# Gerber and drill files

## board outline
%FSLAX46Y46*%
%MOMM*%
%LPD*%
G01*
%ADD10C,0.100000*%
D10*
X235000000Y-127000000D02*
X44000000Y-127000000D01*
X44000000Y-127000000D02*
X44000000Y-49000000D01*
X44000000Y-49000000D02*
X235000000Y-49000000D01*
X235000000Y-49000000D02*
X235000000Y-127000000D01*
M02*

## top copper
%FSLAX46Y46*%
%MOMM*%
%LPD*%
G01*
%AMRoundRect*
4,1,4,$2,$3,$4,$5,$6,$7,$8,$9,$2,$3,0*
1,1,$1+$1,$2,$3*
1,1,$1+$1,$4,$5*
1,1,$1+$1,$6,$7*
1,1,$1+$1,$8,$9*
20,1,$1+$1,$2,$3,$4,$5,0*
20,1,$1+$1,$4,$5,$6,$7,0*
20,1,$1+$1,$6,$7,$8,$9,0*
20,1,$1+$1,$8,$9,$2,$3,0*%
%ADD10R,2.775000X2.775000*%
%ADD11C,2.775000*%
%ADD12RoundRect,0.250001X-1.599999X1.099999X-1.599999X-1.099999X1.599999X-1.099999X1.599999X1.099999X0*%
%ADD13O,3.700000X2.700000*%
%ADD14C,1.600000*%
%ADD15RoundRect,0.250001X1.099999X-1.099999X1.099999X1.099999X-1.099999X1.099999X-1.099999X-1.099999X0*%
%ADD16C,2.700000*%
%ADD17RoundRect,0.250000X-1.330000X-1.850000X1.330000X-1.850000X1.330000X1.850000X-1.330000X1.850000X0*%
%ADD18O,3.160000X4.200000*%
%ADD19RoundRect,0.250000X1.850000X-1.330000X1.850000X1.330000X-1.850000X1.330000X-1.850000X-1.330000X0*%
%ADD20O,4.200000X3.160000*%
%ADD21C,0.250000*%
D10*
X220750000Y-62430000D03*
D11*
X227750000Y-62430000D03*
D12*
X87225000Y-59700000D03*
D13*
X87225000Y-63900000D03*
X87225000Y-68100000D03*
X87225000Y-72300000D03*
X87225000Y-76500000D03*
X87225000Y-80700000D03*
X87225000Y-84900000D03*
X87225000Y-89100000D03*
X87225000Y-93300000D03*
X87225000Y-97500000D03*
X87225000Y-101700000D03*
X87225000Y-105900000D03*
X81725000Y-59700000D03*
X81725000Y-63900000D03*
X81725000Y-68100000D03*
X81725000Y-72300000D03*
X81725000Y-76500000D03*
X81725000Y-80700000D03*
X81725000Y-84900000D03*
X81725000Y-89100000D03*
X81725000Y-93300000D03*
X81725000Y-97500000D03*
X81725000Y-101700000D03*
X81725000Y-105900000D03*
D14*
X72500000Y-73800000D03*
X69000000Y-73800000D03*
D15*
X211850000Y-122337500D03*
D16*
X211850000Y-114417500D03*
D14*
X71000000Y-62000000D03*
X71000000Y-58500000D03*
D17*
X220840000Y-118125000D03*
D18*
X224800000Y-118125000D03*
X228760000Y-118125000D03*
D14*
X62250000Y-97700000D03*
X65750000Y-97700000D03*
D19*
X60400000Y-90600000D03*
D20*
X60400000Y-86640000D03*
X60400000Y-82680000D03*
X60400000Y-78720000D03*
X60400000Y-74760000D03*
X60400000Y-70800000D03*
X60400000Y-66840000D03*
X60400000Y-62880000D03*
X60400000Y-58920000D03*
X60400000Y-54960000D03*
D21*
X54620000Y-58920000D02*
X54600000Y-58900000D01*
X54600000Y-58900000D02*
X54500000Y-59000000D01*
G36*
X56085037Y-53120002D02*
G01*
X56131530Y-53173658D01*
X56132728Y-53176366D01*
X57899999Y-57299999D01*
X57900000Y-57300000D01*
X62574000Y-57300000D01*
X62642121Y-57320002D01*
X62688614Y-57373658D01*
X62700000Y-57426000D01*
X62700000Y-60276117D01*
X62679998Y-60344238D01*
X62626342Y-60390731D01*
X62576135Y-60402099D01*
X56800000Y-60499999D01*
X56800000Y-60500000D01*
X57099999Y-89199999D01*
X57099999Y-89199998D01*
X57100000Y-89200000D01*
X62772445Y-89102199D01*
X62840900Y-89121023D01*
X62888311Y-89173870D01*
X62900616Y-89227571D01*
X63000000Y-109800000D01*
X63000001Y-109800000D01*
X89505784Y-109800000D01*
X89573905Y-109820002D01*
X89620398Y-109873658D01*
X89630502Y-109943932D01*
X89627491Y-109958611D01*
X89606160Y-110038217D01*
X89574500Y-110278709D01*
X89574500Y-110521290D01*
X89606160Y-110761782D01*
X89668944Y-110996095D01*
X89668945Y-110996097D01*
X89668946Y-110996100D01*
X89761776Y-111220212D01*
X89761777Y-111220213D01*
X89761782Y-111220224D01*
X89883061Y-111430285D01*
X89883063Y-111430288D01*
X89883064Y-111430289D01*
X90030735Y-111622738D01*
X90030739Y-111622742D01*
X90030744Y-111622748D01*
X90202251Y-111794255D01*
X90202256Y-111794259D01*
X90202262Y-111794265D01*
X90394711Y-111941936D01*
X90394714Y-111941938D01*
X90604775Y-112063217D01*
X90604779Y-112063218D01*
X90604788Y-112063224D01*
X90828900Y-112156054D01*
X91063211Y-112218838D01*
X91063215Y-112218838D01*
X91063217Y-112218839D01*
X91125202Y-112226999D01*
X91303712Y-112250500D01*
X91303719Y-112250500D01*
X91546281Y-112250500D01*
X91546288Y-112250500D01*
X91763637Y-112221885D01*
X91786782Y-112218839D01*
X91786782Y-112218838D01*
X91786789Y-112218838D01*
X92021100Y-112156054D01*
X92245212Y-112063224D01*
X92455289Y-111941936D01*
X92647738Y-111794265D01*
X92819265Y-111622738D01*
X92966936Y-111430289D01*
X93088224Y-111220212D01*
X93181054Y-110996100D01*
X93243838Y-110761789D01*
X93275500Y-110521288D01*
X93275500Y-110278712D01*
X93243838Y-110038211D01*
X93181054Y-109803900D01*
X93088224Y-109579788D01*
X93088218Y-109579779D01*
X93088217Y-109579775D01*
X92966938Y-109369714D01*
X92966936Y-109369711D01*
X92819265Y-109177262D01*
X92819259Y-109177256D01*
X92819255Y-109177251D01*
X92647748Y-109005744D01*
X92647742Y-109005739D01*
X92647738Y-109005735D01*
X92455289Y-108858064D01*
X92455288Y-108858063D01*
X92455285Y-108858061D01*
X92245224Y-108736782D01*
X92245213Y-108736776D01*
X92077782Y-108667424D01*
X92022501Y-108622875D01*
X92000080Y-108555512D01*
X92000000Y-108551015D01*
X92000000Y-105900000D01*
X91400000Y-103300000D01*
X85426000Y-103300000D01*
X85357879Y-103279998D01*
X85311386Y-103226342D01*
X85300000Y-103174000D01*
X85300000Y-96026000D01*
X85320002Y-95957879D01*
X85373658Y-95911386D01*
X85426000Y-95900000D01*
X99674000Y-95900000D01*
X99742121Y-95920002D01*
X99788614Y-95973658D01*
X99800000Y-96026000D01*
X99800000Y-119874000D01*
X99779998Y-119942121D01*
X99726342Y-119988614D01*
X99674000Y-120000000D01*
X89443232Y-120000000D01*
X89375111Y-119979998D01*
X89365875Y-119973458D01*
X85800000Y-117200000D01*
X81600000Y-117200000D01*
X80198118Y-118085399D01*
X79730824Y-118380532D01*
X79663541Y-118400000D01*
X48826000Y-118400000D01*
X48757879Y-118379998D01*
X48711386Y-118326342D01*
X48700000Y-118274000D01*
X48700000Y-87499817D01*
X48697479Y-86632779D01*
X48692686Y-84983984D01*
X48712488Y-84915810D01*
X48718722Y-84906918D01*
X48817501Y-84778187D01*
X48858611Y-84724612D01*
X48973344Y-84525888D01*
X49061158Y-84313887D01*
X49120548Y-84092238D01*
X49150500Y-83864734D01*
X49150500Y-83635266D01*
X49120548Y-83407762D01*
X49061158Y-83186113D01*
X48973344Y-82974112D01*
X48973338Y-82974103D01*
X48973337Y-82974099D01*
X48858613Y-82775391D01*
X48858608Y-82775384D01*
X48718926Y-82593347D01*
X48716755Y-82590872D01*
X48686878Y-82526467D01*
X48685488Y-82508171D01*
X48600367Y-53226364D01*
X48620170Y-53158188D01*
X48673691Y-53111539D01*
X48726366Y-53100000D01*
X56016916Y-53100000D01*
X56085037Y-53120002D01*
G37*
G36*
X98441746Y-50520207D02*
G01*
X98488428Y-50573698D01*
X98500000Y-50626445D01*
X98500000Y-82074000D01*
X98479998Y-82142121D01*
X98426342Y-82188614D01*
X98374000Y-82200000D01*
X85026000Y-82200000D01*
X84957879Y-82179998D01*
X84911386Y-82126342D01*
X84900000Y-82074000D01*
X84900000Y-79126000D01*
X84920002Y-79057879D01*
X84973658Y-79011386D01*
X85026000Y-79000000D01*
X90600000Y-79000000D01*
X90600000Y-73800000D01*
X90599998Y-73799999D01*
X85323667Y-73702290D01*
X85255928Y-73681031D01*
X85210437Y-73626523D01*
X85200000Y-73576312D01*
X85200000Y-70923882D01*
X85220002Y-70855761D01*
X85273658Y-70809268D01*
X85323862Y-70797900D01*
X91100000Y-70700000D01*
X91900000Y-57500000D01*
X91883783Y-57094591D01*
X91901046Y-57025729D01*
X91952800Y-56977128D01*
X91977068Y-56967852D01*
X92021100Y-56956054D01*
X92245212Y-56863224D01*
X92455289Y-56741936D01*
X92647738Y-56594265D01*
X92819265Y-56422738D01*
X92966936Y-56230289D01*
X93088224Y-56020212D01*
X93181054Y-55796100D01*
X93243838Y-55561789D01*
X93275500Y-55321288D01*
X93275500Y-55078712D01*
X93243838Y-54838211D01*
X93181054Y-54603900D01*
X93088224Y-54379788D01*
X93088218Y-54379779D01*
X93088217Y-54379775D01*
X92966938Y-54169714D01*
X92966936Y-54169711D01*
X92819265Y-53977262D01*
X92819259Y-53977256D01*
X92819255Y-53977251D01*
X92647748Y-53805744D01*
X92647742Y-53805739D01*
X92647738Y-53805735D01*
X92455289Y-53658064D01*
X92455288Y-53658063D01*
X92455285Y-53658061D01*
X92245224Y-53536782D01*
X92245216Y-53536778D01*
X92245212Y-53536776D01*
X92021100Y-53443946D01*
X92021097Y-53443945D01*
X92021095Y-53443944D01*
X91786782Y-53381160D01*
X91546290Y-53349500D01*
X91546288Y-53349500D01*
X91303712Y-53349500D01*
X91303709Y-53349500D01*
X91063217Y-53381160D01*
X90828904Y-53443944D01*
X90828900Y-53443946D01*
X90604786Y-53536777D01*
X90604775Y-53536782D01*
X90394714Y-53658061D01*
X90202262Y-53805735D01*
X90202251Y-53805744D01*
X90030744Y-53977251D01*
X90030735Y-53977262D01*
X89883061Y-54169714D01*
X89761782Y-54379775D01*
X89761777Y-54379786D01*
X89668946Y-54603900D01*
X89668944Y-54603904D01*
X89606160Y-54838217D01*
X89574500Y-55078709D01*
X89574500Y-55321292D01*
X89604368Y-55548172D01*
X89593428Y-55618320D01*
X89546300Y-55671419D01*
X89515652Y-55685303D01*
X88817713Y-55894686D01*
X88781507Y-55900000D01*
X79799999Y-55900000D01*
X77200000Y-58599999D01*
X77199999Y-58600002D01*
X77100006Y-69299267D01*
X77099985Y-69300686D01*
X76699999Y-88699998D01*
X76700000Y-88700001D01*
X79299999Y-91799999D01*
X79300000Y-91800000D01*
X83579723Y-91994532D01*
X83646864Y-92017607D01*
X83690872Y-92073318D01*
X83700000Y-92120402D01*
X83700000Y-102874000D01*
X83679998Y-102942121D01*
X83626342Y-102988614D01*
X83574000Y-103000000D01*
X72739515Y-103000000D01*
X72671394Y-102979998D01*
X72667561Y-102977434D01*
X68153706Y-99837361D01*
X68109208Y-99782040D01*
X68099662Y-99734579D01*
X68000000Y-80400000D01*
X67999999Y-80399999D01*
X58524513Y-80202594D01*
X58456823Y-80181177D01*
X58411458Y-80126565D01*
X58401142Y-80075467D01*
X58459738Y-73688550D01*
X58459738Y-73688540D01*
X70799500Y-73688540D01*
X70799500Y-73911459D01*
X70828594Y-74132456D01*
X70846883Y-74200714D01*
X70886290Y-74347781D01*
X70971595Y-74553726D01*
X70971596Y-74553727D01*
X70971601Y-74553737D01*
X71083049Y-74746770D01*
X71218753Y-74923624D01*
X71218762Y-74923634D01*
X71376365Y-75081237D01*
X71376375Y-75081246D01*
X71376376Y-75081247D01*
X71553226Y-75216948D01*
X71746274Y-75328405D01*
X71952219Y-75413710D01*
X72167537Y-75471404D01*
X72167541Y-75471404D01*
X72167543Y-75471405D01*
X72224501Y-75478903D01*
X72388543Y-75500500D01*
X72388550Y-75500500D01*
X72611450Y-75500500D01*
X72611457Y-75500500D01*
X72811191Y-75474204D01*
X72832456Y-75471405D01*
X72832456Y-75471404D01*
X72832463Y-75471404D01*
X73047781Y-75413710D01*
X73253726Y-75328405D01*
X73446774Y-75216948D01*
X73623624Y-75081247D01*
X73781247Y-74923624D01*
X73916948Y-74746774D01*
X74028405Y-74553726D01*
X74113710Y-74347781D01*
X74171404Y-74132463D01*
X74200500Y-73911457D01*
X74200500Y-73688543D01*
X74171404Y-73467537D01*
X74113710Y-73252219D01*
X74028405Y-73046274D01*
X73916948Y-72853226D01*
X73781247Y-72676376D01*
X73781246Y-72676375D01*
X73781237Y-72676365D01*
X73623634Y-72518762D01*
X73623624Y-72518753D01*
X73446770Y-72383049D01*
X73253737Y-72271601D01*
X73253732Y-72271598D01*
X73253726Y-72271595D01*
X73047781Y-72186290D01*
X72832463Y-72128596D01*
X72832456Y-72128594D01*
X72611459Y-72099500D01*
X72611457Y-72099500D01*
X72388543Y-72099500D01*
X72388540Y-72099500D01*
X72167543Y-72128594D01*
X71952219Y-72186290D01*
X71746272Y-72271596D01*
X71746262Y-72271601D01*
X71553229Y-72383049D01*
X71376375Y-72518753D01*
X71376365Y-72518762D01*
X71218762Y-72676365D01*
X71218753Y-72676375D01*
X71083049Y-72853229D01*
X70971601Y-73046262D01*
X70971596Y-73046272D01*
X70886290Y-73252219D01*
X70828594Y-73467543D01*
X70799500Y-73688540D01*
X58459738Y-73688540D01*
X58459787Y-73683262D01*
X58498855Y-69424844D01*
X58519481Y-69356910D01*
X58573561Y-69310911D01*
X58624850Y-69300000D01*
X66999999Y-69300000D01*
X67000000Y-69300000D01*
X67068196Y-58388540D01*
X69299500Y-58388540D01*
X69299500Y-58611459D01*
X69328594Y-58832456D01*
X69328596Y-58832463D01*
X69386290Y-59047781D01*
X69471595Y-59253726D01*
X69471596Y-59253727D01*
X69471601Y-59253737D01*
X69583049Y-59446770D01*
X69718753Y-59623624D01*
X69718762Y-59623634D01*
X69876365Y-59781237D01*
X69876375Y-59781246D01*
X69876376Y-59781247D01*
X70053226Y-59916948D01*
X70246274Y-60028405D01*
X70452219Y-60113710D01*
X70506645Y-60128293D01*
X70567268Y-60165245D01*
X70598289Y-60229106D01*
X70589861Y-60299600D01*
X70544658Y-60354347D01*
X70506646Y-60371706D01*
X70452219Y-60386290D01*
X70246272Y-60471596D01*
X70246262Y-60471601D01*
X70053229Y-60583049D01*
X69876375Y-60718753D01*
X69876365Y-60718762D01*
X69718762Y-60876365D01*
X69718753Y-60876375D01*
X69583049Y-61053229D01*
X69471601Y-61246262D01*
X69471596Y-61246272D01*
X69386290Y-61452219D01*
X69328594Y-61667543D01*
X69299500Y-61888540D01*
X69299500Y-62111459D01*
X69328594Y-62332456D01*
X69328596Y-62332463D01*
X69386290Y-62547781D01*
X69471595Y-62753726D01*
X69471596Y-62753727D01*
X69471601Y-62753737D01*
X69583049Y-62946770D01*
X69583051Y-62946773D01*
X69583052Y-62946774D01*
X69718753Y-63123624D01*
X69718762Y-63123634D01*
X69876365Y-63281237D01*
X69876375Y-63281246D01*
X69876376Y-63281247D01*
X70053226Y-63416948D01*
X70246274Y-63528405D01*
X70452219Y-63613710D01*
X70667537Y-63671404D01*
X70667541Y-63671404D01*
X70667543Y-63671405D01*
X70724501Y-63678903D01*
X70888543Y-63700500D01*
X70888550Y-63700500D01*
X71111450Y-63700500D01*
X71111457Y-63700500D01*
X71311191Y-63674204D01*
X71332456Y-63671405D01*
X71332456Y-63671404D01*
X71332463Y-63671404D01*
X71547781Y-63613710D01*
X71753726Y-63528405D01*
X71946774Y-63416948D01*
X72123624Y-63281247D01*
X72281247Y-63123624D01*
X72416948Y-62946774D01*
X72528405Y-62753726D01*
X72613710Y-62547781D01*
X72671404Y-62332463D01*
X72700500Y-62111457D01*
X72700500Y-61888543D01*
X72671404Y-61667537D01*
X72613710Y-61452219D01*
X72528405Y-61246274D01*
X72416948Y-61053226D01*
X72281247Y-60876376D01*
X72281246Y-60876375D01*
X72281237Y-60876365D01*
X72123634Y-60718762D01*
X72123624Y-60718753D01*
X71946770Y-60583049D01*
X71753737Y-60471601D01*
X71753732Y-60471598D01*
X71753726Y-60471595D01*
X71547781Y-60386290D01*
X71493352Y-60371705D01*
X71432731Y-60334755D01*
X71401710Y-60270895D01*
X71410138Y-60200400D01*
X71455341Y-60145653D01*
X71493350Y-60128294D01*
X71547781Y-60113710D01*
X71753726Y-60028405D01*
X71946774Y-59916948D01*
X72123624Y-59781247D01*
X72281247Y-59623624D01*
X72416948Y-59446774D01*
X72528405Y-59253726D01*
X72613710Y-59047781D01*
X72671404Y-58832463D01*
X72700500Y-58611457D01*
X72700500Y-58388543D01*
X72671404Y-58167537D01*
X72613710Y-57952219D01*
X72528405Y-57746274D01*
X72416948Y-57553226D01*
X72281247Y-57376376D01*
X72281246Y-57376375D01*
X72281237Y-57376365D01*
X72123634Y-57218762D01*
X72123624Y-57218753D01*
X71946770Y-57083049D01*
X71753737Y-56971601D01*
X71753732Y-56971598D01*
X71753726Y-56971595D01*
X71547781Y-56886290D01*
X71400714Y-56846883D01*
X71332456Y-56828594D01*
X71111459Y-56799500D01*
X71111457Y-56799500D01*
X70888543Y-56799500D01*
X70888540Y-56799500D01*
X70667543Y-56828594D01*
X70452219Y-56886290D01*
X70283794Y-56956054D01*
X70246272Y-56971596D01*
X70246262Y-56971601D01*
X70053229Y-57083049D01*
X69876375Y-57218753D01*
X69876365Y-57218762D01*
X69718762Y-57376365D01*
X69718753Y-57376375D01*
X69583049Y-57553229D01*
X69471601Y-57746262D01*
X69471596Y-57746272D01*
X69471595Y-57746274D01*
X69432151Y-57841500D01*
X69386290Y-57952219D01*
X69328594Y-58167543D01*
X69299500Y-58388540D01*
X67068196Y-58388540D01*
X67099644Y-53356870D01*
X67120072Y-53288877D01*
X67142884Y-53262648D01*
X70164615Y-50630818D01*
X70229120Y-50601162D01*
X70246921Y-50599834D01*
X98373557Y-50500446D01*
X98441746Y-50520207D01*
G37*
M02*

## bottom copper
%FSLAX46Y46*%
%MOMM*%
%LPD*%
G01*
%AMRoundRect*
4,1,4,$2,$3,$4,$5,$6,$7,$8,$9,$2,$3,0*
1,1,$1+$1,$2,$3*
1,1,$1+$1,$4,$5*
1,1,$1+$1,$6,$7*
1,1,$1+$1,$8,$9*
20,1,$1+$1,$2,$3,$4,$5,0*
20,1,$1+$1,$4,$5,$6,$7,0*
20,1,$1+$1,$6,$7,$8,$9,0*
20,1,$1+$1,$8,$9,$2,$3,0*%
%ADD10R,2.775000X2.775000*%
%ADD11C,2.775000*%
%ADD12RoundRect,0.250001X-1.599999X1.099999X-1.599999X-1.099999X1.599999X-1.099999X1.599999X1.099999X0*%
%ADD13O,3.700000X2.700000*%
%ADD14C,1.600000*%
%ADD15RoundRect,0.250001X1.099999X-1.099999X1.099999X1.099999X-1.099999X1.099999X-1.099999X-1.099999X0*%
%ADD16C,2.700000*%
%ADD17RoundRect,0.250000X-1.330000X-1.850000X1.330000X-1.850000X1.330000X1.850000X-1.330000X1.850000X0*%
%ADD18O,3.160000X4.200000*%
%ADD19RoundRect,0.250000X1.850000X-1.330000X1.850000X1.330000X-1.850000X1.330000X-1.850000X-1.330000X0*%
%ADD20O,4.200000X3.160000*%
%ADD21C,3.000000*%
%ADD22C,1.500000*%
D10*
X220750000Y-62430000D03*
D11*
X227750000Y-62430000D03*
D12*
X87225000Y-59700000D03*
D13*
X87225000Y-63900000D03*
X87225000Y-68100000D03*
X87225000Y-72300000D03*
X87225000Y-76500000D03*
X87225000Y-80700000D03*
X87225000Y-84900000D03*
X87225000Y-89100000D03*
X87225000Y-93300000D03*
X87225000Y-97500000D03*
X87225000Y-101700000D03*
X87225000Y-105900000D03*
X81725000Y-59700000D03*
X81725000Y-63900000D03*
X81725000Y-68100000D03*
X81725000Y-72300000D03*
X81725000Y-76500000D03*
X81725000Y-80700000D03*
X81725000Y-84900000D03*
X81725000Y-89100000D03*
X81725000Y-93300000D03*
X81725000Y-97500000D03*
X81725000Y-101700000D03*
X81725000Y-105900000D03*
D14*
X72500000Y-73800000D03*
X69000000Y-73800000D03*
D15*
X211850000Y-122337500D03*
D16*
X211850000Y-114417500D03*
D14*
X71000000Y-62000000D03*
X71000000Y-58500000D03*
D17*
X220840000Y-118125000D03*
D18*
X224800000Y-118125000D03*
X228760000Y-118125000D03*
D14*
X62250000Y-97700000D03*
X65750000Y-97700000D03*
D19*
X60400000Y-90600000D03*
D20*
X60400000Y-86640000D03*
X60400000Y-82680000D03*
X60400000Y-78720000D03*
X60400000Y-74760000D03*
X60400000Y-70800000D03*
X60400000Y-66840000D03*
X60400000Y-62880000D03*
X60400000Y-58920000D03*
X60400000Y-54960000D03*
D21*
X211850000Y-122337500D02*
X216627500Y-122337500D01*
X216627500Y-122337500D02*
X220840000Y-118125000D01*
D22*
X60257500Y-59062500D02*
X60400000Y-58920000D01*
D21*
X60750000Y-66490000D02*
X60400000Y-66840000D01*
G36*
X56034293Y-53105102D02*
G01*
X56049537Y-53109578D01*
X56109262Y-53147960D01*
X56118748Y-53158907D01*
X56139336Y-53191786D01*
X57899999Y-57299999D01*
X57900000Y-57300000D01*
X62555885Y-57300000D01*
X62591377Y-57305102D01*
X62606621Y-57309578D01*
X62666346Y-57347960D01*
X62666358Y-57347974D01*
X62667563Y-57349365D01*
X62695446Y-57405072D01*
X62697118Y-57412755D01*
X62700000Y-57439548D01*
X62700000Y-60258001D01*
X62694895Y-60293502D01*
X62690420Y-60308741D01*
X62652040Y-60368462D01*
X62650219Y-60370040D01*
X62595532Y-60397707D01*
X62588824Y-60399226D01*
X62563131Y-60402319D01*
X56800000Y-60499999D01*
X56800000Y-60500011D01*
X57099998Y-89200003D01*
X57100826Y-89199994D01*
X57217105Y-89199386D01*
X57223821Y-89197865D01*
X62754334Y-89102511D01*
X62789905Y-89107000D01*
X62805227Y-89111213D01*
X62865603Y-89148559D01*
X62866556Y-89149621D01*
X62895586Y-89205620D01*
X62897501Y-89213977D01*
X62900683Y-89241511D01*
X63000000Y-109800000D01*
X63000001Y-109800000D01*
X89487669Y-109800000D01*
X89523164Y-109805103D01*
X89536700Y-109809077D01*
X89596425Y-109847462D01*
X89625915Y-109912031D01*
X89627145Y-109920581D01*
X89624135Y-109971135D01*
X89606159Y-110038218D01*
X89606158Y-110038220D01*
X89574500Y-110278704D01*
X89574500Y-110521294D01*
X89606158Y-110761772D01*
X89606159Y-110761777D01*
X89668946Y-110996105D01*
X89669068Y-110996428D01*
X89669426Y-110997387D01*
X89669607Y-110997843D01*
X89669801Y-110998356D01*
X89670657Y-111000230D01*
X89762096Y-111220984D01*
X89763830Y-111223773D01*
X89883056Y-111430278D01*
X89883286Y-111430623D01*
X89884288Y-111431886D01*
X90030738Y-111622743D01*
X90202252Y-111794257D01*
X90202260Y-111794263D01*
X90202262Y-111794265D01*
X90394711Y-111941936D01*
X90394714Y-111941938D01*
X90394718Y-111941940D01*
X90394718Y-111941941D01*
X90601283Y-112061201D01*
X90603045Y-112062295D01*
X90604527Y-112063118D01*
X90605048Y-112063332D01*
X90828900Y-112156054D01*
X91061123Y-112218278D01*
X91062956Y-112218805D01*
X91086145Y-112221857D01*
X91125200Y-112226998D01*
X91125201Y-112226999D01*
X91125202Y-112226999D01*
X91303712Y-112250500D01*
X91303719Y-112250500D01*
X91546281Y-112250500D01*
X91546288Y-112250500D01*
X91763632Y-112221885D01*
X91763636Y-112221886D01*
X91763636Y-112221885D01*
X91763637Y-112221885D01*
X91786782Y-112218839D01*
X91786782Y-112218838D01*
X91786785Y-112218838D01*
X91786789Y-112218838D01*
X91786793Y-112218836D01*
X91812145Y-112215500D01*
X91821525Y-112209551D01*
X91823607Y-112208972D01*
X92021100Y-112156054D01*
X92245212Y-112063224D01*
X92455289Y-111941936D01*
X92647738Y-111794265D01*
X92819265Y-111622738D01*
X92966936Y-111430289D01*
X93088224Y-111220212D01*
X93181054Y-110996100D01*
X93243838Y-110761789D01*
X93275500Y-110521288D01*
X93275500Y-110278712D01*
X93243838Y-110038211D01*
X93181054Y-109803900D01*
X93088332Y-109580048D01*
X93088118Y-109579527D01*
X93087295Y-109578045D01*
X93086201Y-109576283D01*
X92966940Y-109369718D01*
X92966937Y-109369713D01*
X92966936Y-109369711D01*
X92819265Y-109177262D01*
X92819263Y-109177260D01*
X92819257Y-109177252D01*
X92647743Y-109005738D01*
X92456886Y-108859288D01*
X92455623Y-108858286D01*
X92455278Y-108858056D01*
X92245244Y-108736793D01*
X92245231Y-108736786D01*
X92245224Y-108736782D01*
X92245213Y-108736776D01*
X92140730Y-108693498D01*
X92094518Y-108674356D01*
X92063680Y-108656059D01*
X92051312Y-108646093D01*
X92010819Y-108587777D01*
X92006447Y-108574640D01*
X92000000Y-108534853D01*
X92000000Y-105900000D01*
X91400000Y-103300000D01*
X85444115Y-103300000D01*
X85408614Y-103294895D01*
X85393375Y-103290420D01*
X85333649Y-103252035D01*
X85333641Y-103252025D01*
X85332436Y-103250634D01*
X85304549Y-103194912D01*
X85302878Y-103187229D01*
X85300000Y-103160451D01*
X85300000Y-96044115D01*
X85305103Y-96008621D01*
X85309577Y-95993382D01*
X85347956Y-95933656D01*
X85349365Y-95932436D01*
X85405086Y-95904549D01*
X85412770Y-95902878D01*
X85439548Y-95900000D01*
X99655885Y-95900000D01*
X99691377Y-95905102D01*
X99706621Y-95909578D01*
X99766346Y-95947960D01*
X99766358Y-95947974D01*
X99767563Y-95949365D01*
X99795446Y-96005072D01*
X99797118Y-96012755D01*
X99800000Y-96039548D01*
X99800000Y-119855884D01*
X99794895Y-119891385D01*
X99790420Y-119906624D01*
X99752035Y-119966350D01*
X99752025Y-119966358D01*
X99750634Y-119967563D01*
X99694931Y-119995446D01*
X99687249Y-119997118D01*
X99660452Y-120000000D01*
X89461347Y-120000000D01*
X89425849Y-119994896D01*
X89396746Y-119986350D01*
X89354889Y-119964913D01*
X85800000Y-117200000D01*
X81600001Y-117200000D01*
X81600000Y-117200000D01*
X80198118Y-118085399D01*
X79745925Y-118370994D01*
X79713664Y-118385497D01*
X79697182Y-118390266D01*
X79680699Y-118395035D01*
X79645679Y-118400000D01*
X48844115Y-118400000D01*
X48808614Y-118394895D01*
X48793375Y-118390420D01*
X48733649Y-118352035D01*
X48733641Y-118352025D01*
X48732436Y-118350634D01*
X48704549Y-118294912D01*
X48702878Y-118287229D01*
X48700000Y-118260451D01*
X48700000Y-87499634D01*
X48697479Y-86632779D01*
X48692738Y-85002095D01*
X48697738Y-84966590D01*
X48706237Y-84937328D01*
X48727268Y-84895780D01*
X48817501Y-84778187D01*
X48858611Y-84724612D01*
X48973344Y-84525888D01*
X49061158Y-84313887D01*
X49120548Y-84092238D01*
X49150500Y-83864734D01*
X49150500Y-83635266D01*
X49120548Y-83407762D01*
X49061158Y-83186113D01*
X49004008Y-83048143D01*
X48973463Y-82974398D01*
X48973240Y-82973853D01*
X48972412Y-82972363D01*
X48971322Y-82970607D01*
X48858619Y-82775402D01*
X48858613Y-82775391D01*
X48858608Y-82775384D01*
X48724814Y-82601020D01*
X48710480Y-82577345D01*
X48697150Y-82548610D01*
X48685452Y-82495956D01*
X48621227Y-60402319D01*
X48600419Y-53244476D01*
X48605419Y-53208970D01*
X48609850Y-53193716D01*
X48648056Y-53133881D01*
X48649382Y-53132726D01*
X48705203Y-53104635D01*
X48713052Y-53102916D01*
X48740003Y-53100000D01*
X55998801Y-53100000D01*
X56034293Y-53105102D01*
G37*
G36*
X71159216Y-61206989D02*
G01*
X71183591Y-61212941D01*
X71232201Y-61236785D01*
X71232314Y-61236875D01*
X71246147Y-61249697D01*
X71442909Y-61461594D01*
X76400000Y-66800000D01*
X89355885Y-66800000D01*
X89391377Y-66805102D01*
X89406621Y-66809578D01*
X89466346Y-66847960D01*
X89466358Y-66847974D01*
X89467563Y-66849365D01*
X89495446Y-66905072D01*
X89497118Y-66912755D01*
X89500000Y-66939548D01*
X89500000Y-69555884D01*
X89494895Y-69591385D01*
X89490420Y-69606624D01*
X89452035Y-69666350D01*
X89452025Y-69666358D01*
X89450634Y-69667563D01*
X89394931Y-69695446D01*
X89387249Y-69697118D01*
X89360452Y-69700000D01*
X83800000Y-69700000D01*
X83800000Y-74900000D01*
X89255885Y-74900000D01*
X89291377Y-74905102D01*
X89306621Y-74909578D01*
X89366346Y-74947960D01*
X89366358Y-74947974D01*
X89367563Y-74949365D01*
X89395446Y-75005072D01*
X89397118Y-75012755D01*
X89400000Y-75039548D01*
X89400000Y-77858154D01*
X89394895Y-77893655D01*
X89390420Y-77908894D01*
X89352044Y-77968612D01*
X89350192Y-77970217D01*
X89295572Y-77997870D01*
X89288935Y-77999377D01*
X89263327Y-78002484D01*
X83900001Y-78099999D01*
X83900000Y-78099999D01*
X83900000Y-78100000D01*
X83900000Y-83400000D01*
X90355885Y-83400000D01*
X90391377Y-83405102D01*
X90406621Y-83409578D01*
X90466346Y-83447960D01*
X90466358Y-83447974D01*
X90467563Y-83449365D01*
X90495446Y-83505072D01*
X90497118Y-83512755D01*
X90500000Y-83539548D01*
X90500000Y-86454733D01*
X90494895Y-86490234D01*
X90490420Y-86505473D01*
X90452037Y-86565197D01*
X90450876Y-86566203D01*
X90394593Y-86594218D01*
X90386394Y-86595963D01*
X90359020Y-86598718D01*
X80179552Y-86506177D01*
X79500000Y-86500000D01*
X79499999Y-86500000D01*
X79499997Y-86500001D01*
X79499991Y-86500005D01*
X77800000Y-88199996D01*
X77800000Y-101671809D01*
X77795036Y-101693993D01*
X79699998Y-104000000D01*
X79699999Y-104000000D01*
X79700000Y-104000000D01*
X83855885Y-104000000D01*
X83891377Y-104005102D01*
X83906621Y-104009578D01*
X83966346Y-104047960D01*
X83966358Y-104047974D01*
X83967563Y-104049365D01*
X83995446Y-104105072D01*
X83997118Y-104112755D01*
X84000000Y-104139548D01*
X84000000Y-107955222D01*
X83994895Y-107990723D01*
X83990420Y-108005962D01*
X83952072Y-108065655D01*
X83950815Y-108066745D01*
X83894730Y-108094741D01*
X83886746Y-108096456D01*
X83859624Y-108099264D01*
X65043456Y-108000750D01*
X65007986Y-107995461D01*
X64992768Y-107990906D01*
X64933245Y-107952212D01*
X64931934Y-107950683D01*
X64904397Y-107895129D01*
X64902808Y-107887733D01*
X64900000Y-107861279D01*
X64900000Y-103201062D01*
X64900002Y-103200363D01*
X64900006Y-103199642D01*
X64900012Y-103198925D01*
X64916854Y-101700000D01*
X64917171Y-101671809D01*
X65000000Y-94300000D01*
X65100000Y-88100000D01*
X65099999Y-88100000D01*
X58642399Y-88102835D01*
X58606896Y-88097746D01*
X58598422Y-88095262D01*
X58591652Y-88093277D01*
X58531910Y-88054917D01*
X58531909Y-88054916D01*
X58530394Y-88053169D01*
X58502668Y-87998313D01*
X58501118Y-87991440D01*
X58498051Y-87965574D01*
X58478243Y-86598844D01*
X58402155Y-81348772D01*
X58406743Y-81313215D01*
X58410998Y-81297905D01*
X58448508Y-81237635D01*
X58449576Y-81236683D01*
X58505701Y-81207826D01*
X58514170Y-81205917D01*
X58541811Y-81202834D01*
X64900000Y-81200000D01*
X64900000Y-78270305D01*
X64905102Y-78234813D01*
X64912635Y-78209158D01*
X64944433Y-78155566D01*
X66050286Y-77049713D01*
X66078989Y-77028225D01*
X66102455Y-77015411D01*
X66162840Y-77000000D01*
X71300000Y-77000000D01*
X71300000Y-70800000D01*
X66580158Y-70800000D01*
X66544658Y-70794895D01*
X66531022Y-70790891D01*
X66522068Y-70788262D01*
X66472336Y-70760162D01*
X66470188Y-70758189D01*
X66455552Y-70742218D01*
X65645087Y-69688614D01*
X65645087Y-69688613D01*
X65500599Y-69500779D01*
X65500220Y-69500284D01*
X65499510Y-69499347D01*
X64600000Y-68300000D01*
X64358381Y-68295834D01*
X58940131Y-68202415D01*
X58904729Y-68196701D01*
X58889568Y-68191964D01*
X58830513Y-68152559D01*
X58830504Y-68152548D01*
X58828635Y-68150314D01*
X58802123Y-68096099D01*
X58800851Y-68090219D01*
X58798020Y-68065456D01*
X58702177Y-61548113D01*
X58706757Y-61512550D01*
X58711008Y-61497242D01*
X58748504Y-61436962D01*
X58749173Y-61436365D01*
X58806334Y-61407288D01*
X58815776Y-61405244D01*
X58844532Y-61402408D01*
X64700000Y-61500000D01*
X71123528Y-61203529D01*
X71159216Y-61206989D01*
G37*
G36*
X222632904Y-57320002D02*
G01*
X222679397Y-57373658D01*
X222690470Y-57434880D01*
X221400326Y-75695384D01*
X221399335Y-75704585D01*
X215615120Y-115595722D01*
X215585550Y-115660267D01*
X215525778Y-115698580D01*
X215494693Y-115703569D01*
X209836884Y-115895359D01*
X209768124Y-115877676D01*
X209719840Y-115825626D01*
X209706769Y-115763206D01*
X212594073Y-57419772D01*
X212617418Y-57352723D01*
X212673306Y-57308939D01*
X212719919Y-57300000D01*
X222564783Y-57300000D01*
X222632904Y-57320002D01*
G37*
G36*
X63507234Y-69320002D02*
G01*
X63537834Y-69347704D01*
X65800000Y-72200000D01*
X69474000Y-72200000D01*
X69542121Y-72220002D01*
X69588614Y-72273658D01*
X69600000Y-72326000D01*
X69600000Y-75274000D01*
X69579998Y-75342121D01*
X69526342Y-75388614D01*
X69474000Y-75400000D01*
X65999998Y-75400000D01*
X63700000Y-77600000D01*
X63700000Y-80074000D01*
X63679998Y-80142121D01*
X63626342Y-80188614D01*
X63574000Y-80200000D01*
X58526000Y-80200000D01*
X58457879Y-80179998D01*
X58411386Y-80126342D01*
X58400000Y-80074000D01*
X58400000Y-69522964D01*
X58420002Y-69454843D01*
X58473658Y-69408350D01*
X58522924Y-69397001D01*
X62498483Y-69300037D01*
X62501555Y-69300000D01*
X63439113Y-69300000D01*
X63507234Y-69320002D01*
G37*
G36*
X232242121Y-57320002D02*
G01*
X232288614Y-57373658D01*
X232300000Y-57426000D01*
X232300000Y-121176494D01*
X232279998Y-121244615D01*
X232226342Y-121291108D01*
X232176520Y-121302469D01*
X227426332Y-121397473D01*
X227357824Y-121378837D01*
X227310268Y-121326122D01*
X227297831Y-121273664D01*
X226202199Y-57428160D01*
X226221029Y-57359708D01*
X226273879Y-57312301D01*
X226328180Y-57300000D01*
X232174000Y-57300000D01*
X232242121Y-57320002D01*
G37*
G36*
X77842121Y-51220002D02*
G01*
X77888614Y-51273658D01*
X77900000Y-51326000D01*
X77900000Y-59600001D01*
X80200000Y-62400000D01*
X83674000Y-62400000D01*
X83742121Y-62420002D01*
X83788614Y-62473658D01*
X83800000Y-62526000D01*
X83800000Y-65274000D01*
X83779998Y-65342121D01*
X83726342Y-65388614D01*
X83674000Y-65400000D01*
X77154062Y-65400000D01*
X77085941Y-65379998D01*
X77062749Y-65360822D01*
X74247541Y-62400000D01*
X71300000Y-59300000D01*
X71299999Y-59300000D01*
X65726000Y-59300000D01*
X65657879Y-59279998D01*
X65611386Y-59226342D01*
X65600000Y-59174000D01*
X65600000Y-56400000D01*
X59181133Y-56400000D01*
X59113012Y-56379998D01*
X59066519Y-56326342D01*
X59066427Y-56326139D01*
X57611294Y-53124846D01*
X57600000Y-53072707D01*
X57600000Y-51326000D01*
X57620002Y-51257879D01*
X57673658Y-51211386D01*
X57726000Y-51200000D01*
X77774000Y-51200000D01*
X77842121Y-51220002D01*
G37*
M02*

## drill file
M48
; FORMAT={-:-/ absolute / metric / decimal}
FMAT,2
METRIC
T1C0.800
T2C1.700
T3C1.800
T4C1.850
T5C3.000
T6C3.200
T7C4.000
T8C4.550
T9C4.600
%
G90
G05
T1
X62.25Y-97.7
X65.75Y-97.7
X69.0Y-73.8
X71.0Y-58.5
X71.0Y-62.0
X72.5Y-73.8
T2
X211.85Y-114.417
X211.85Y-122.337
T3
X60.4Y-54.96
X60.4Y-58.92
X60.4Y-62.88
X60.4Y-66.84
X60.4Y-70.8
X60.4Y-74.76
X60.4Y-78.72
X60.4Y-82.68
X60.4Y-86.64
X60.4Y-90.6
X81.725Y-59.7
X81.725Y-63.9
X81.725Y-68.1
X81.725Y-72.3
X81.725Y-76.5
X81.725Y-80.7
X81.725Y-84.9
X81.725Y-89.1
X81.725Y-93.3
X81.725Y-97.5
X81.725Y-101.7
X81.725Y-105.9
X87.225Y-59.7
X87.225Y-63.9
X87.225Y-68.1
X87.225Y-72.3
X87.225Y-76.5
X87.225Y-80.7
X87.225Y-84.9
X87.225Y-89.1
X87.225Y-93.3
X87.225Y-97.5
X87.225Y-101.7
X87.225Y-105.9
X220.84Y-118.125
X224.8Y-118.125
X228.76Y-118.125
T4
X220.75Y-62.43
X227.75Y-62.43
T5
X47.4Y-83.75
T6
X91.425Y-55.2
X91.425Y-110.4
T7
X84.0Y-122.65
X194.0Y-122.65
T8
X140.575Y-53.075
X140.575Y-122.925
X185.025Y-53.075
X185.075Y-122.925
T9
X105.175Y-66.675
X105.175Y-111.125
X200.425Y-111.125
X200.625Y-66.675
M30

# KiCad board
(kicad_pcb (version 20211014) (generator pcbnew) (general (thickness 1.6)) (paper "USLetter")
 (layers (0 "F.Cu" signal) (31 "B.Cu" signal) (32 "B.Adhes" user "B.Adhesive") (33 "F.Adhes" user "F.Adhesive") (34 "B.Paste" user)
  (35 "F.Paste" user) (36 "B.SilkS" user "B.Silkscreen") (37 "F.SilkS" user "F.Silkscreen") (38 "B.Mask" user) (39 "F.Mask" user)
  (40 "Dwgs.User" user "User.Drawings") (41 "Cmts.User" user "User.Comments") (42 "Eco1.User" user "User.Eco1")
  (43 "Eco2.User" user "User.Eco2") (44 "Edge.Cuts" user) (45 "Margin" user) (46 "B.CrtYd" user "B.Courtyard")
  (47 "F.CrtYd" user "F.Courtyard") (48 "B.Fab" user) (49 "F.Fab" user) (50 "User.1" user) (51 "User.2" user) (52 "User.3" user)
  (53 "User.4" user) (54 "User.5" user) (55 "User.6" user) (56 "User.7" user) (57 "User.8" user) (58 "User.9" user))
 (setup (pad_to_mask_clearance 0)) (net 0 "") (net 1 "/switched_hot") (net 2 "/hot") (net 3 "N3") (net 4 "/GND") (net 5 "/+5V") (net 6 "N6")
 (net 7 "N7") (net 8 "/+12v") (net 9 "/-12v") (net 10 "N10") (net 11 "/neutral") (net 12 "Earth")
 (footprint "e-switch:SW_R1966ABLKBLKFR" (layer "F.Cu") (at 220.75 62.43)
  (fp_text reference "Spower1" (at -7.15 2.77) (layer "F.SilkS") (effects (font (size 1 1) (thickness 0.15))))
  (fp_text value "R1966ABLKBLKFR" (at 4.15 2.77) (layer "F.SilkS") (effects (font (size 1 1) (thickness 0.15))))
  (pad "1" thru_hole rect locked (at 0 0) (size 2.775 2.775) (drill 1.85) (layers *.Cu *.Mask) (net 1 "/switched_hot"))
  (pad "1A" thru_hole circle locked (at 7 0) (size 2.775 2.775) (drill 1.85) (layers *.Cu *.Mask) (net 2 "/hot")))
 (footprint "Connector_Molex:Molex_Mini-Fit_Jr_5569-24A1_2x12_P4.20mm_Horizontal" (layer "F.Cu") (at 87.225 59.7 -90)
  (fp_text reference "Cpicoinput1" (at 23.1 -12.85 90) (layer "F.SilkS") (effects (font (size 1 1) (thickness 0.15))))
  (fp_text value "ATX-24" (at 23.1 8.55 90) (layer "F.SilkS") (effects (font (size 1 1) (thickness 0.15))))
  (pad "" np_thru_hole circle (at -4.5 -4.2 270) (size 3.2 3.2) (drill 3.2) (layers F&B.Cu *.Mask))
  (pad "" np_thru_hole circle (at 50.7 -4.2 270) (size 3.2 3.2) (drill 3.2) (layers *.Cu *.Mask))
  (pad "1" thru_hole roundrect (at 0 0 270) (size 2.7 3.7) (drill 1.8) (layers *.Cu *.Mask) (roundrect_rratio 0.09259296296) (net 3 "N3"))
  (pad "2" thru_hole oval (at 4.2 0 270) (size 2.7 3.7) (drill 1.8) (layers *.Cu *.Mask) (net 3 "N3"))
  (pad "3" thru_hole oval (at 8.4 0 270) (size 2.7 3.7) (drill 1.8) (layers *.Cu *.Mask) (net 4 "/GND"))
  (pad "4" thru_hole oval (at 12.6 0 270) (size 2.7 3.7) (drill 1.8) (layers *.Cu *.Mask) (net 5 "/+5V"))
  (pad "5" thru_hole oval (at 16.8 0 270) (size 2.7 3.7) (drill 1.8) (layers *.Cu *.Mask) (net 4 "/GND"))
  (pad "6" thru_hole oval (at 21 0 270) (size 2.7 3.7) (drill 1.8) (layers *.Cu *.Mask) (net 5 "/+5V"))
  (pad "7" thru_hole oval (at 25.2 0 270) (size 2.7 3.7) (drill 1.8) (layers *.Cu *.Mask) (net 4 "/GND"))
  (pad "8" thru_hole oval (at 29.4 0 270) (size 2.7 3.7) (drill 1.8) (layers *.Cu *.Mask) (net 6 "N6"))
  (pad "9" thru_hole oval (at 33.6 0 270) (size 2.7 3.7) (drill 1.8) (layers *.Cu *.Mask) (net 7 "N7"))
  (pad "10" thru_hole oval (at 37.8 0 270) (size 2.7 3.7) (drill 1.8) (layers *.Cu *.Mask) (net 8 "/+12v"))
  (pad "11" thru_hole oval (at 42 0 270) (size 2.7 3.7) (drill 1.8) (layers *.Cu *.Mask) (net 8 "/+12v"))
  (pad "12" thru_hole oval (at 46.2 0 270) (size 2.7 3.7) (drill 1.8) (layers *.Cu *.Mask) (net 3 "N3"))
  (pad "13" thru_hole oval (at 0 5.5 270) (size 2.7 3.7) (drill 1.8) (layers *.Cu *.Mask) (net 3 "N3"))
  (pad "14" thru_hole oval (at 4.2 5.5 270) (size 2.7 3.7) (drill 1.8) (layers *.Cu *.Mask) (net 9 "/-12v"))
  (pad "15" thru_hole oval (at 8.4 5.5 270) (size 2.7 3.7) (drill 1.8) (layers *.Cu *.Mask) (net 4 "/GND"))
  (pad "16" thru_hole oval (at 12.6 5.5 270) (size 2.7 3.7) (drill 1.8) (layers *.Cu *.Mask) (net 4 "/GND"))
  (pad "17" thru_hole oval (at 16.8 5.5 270) (size 2.7 3.7) (drill 1.8) (layers *.Cu *.Mask) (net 4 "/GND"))
  (pad "18" thru_hole oval (at 21 5.5 270) (size 2.7 3.7) (drill 1.8) (layers *.Cu *.Mask) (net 4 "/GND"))
  (pad "19" thru_hole oval (at 25.2 5.5 270) (size 2.7 3.7) (drill 1.8) (layers *.Cu *.Mask) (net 4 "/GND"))
  (pad "20" thru_hole oval (at 29.4 5.5 270) (size 2.7 3.7) (drill 1.8) (layers *.Cu *.Mask) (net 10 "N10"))
  (pad "21" thru_hole oval (at 33.6 5.5 270) (size 2.7 3.7) (drill 1.8) (layers *.Cu *.Mask) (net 5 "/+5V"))
  (pad "22" thru_hole oval (at 37.8 5.5 270) (size 2.7 3.7) (drill 1.8) (layers *.Cu *.Mask) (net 5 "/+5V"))
  (pad "23" thru_hole oval (at 42 5.5 270) (size 2.7 3.7) (drill 1.8) (layers *.Cu *.Mask) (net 5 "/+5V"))
  (pad "24" thru_hole oval (at 46.2 5.5 270) (size 2.7 3.7) (drill 1.8) (layers *.Cu *.Mask) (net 4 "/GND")))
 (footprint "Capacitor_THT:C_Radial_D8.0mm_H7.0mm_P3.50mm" (layer "F.Cu") (at 72.5 73.8 180)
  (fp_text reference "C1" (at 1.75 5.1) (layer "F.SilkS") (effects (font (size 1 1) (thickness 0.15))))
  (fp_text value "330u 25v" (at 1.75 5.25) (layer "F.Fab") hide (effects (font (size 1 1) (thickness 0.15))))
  (pad "1" thru_hole circle (at 0 0 180) (size 1.6 1.6) (drill 0.8) (layers *.Cu *.Mask) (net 4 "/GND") (clearance 0.9))
  (pad "2" thru_hole circle (at 3.5 0 180) (size 1.6 1.6) (drill 0.8) (layers *.Cu *.Mask) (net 5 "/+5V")))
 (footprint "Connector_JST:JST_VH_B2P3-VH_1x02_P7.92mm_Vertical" (layer "F.Cu") (at 211.85 122.3375 90)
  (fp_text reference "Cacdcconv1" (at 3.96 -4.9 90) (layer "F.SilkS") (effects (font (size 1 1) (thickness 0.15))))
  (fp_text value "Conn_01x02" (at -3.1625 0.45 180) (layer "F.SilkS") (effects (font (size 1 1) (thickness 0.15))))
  (pad "1" thru_hole roundrect (at 0 0 90) (size 2.7 2.7) (drill 1.7) (layers *.Cu *.Mask) (roundrect_rratio 0.09259296296)
   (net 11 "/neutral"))
  (pad "2" thru_hole circle (at 7.92 0 90) (size 2.7 2.7) (drill 1.7) (layers *.Cu *.Mask) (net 1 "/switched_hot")))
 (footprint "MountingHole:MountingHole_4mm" (layer "F.Cu") (at 84 122.65)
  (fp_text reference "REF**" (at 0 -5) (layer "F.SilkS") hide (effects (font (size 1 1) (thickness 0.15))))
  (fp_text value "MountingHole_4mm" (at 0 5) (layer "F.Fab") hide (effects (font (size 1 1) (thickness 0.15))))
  (pad "" np_thru_hole circle (at 0 0) (size 4 4) (drill 4) (layers *.Cu *.Mask)))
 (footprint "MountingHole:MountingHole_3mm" (layer "F.Cu") (at 47.4 83.75)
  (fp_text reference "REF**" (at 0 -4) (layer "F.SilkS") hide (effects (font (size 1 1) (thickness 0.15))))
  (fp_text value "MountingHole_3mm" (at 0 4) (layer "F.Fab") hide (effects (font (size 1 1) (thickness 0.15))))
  (pad "" np_thru_hole circle (at 0 0) (size 3 3) (drill 3) (layers *.Cu *.Mask)))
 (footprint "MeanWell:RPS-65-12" (layer "F.Cu") (at 188.2 49.9 -90)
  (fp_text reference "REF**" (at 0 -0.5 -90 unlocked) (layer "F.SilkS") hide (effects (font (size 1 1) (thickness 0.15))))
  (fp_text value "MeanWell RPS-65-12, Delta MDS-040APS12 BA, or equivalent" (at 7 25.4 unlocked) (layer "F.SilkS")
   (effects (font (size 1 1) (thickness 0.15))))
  (pad "" np_thru_hole circle (at 73.025 47.625 270) (size 4.55 4.55) (drill 4.55) (layers F&B.Cu *.Mask))
  (pad "" np_thru_hole circle (at 73.025 3.125 270) (size 4.55 4.55) (drill 4.55) (layers F&B.Cu *.Mask))
  (pad "" np_thru_hole circle (at 3.175 3.175 270) (size 4.55 4.55) (drill 4.55) (layers F&B.Cu *.Mask))
  (pad "" np_thru_hole circle (at 3.175 47.625 270) (size 4.55 4.55) (drill 4.55) (layers F&B.Cu *.Mask)))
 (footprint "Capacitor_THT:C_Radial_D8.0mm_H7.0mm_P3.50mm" (layer "F.Cu") (at 71 62 90)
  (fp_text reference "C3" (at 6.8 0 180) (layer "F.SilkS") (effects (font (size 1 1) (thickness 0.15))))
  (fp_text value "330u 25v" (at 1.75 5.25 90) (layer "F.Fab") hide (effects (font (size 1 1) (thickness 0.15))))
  (pad "1" thru_hole circle (at 0 0 90) (size 1.6 1.6) (drill 0.8) (layers *.Cu *.Mask) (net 4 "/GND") (clearance 0.9))
  (pad "2" thru_hole circle (at 3.5 0 90) (size 1.6 1.6) (drill 0.8) (layers *.Cu *.Mask) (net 9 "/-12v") (clearance 0.9)))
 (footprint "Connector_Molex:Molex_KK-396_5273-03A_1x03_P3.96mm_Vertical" (layer "F.Cu") (at 220.84 118.125)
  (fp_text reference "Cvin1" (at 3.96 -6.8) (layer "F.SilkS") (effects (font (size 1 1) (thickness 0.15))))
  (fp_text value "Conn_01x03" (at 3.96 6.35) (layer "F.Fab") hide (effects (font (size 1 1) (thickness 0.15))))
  (pad "1" thru_hole roundrect (at 0 0) (size 3.16 4.2) (drill 1.8) (layers *.Cu *.Mask) (roundrect_rratio 0.07911392405)
   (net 11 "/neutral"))
  (pad "2" thru_hole oval (at 3.96 0) (size 3.16 4.2) (drill 1.8) (layers *.Cu *.Mask) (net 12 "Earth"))
  (pad "3" thru_hole oval (at 7.92 0) (size 3.16 4.2) (drill 1.8) (layers *.Cu *.Mask) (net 2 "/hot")))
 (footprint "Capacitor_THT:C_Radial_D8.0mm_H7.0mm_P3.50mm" (layer "F.Cu") (at 62.25 97.7)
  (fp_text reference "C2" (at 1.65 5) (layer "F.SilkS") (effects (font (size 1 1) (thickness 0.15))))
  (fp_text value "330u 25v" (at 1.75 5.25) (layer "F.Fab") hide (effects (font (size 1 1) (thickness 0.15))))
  (pad "1" thru_hole circle (at 0 0) (size 1.6 1.6) (drill 0.8) (layers *.Cu *.Mask) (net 8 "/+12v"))
  (pad "2" thru_hole circle (at 3.5 0) (size 1.6 1.6) (drill 0.8) (layers *.Cu *.Mask) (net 4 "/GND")))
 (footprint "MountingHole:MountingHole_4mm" (layer "F.Cu") (at 194 122.65)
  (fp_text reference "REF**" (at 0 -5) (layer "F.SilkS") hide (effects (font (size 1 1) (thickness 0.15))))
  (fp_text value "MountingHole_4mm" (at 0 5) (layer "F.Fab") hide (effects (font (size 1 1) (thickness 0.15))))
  (pad "" np_thru_hole circle (at 0 0) (size 4 4) (drill 4) (layers *.Cu *.Mask)))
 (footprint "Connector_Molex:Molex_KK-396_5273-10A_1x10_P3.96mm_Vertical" (layer "F.Cu") (at 60.4 90.6 90)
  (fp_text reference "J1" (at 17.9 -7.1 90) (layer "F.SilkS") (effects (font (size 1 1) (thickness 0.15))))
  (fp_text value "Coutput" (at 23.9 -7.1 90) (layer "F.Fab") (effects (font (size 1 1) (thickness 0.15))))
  (pad "1" thru_hole roundrect (at 0 0 90) (size 3.16 4.2) (drill 1.8) (layers *.Cu *.Mask) (roundrect_rratio 0.07911392405) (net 8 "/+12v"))
  (pad "2" thru_hole oval (at 3.96 0 90) (size 3.16 4.2) (drill 1.8) (layers *.Cu *.Mask) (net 4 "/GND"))
  (pad "3" thru_hole oval (at 7.92 0 90) (size 3.16 4.2) (drill 1.8) (layers *.Cu *.Mask) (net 4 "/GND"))
  (pad "4" thru_hole oval (at 11.88 0 90) (size 3.16 4.2) (drill 1.8) (layers *.Cu *.Mask) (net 5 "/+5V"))
  (pad "5" thru_hole oval (at 15.84 0 90) (size 3.16 4.2) (drill 1.8) (layers *.Cu *.Mask) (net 5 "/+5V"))
  (pad "6" thru_hole oval (at 19.8 0 90) (size 3.16 4.2) (drill 1.8) (layers *.Cu *.Mask) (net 5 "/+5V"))
  (pad "7" thru_hole oval (at 23.76 0 90) (size 3.16 4.2) (drill 1.8) (layers *.Cu *.Mask) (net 4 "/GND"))
  (pad "8" thru_hole oval (at 27.72 0 90) (size 3.16 4.2) (drill 1.8) (layers *.Cu *.Mask) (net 4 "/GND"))
  (pad "9" thru_hole oval (at 31.68 0 90) (size 3.16 4.2) (drill 1.8) (layers *.Cu *.Mask) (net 8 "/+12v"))
  (pad "10" thru_hole oval (at 35.64 0 90) (size 3.16 4.2) (drill 1.8) (layers *.Cu *.Mask) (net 9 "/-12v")))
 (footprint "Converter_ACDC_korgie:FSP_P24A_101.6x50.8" (layer "F.Cu") (at 102 63.5)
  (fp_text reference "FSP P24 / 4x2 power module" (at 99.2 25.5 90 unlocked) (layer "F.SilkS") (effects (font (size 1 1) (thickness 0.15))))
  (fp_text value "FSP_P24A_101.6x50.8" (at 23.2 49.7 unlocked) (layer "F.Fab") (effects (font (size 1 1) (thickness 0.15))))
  (pad "" np_thru_hole circle (at 3.175 47.625) (size 4.6 4.6) (drill 4.6) (layers F&B.Cu *.Mask))
  (pad "" np_thru_hole circle (at 98.425 47.625) (size 4.6 4.6) (drill 4.6) (layers F&B.Cu *.Mask))
  (pad "" np_thru_hole circle (at 98.625 3.175) (size 4.6 4.6) (drill 4.6) (layers F&B.Cu *.Mask))
  (pad "" np_thru_hole circle (at 3.175 3.175) (size 4.6 4.6) (drill 4.6) (layers F&B.Cu *.Mask)))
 (gr_line (start 235 127) (end 44 127) (layer "Edge.Cuts") (width 0.1))
 (gr_line (start 44 127) (end 44 49) (layer "Edge.Cuts") (width 0.1))
 (gr_line (start 44 49) (end 235 49) (layer "Edge.Cuts") (width 0.1))
 (gr_line (start 235 49) (end 235 127) (layer "Edge.Cuts") (width 0.1))
 (segment (start 211.85 122.3375) (end 216.6275 122.3375) (width 3) (layer "B.Cu") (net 11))
 (segment (start 216.6275 122.3375) (end 220.84 118.125) (width 3) (layer "B.Cu") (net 11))
 (segment (start 54.62 58.92) (end 54.6 58.9) (width 0.25) (layer "F.Cu") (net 8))
 (segment (start 54.6 58.9) (end 54.5 59) (width 0.25) (layer "F.Cu") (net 8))
 (segment (start 60.2575 59.0625) (end 60.4 58.92) (width 1.5) (layer "B.Cu") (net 8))
 (segment (start 60.75 66.49) (end 60.4 66.84) (width 3) (layer "B.Cu") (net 4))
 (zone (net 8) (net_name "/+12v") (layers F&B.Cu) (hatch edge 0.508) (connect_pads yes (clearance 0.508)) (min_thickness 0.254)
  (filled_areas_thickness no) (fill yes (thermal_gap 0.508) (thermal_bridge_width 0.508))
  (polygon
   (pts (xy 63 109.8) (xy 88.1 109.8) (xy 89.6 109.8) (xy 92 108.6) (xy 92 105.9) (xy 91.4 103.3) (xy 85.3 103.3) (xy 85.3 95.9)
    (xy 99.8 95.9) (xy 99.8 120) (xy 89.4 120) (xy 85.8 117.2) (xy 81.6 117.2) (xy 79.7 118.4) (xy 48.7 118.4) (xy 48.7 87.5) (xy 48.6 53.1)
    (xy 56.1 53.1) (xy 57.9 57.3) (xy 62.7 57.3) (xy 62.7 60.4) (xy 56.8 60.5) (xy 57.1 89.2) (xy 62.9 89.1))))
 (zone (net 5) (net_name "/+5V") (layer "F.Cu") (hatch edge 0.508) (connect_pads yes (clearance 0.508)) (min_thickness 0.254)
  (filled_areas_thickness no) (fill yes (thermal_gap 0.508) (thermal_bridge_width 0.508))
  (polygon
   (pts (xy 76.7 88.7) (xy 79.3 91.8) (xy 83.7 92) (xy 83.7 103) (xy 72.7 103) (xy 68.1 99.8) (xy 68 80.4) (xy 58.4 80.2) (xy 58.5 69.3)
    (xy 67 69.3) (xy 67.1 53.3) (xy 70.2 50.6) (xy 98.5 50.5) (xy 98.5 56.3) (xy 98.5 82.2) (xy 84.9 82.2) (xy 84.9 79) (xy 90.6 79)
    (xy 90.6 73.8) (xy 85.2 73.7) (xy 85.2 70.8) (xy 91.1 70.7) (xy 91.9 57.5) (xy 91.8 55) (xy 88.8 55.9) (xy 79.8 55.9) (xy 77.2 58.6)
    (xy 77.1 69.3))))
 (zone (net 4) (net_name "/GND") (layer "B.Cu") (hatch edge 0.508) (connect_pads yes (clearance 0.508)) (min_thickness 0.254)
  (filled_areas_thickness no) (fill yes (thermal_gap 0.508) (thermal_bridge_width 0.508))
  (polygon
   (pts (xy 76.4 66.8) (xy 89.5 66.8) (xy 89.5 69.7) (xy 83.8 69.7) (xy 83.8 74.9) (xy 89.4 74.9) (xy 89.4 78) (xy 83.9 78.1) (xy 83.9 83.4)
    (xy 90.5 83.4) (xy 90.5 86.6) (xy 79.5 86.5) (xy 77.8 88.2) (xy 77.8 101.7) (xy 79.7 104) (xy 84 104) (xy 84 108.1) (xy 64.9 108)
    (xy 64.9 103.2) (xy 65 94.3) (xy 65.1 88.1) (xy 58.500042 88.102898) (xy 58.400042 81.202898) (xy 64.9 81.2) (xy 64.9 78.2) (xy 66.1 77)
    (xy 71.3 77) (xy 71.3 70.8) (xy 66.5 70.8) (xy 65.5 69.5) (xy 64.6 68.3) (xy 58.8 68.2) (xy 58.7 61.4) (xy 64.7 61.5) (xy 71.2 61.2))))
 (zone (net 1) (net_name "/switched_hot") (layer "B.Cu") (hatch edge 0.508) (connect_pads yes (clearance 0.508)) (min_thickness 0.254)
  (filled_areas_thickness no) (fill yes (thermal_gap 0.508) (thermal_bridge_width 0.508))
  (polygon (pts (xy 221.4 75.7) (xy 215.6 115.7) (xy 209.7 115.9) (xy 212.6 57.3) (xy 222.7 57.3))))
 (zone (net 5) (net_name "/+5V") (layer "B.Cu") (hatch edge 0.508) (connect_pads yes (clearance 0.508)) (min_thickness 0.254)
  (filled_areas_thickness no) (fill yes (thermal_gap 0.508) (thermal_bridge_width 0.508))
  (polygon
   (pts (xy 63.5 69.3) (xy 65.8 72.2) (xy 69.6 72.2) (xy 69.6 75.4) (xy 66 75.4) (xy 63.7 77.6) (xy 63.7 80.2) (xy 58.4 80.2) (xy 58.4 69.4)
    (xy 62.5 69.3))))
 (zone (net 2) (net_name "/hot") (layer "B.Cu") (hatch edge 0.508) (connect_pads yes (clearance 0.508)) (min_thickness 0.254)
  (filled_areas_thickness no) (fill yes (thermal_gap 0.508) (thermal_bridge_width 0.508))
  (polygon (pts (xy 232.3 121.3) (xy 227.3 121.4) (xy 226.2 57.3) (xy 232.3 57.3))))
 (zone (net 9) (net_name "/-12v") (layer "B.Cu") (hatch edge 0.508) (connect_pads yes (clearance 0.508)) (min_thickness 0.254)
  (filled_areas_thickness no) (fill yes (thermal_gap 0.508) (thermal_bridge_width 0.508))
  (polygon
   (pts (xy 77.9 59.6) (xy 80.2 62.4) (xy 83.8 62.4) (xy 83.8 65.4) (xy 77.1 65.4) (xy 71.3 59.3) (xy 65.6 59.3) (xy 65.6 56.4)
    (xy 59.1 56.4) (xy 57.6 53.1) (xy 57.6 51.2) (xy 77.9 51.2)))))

